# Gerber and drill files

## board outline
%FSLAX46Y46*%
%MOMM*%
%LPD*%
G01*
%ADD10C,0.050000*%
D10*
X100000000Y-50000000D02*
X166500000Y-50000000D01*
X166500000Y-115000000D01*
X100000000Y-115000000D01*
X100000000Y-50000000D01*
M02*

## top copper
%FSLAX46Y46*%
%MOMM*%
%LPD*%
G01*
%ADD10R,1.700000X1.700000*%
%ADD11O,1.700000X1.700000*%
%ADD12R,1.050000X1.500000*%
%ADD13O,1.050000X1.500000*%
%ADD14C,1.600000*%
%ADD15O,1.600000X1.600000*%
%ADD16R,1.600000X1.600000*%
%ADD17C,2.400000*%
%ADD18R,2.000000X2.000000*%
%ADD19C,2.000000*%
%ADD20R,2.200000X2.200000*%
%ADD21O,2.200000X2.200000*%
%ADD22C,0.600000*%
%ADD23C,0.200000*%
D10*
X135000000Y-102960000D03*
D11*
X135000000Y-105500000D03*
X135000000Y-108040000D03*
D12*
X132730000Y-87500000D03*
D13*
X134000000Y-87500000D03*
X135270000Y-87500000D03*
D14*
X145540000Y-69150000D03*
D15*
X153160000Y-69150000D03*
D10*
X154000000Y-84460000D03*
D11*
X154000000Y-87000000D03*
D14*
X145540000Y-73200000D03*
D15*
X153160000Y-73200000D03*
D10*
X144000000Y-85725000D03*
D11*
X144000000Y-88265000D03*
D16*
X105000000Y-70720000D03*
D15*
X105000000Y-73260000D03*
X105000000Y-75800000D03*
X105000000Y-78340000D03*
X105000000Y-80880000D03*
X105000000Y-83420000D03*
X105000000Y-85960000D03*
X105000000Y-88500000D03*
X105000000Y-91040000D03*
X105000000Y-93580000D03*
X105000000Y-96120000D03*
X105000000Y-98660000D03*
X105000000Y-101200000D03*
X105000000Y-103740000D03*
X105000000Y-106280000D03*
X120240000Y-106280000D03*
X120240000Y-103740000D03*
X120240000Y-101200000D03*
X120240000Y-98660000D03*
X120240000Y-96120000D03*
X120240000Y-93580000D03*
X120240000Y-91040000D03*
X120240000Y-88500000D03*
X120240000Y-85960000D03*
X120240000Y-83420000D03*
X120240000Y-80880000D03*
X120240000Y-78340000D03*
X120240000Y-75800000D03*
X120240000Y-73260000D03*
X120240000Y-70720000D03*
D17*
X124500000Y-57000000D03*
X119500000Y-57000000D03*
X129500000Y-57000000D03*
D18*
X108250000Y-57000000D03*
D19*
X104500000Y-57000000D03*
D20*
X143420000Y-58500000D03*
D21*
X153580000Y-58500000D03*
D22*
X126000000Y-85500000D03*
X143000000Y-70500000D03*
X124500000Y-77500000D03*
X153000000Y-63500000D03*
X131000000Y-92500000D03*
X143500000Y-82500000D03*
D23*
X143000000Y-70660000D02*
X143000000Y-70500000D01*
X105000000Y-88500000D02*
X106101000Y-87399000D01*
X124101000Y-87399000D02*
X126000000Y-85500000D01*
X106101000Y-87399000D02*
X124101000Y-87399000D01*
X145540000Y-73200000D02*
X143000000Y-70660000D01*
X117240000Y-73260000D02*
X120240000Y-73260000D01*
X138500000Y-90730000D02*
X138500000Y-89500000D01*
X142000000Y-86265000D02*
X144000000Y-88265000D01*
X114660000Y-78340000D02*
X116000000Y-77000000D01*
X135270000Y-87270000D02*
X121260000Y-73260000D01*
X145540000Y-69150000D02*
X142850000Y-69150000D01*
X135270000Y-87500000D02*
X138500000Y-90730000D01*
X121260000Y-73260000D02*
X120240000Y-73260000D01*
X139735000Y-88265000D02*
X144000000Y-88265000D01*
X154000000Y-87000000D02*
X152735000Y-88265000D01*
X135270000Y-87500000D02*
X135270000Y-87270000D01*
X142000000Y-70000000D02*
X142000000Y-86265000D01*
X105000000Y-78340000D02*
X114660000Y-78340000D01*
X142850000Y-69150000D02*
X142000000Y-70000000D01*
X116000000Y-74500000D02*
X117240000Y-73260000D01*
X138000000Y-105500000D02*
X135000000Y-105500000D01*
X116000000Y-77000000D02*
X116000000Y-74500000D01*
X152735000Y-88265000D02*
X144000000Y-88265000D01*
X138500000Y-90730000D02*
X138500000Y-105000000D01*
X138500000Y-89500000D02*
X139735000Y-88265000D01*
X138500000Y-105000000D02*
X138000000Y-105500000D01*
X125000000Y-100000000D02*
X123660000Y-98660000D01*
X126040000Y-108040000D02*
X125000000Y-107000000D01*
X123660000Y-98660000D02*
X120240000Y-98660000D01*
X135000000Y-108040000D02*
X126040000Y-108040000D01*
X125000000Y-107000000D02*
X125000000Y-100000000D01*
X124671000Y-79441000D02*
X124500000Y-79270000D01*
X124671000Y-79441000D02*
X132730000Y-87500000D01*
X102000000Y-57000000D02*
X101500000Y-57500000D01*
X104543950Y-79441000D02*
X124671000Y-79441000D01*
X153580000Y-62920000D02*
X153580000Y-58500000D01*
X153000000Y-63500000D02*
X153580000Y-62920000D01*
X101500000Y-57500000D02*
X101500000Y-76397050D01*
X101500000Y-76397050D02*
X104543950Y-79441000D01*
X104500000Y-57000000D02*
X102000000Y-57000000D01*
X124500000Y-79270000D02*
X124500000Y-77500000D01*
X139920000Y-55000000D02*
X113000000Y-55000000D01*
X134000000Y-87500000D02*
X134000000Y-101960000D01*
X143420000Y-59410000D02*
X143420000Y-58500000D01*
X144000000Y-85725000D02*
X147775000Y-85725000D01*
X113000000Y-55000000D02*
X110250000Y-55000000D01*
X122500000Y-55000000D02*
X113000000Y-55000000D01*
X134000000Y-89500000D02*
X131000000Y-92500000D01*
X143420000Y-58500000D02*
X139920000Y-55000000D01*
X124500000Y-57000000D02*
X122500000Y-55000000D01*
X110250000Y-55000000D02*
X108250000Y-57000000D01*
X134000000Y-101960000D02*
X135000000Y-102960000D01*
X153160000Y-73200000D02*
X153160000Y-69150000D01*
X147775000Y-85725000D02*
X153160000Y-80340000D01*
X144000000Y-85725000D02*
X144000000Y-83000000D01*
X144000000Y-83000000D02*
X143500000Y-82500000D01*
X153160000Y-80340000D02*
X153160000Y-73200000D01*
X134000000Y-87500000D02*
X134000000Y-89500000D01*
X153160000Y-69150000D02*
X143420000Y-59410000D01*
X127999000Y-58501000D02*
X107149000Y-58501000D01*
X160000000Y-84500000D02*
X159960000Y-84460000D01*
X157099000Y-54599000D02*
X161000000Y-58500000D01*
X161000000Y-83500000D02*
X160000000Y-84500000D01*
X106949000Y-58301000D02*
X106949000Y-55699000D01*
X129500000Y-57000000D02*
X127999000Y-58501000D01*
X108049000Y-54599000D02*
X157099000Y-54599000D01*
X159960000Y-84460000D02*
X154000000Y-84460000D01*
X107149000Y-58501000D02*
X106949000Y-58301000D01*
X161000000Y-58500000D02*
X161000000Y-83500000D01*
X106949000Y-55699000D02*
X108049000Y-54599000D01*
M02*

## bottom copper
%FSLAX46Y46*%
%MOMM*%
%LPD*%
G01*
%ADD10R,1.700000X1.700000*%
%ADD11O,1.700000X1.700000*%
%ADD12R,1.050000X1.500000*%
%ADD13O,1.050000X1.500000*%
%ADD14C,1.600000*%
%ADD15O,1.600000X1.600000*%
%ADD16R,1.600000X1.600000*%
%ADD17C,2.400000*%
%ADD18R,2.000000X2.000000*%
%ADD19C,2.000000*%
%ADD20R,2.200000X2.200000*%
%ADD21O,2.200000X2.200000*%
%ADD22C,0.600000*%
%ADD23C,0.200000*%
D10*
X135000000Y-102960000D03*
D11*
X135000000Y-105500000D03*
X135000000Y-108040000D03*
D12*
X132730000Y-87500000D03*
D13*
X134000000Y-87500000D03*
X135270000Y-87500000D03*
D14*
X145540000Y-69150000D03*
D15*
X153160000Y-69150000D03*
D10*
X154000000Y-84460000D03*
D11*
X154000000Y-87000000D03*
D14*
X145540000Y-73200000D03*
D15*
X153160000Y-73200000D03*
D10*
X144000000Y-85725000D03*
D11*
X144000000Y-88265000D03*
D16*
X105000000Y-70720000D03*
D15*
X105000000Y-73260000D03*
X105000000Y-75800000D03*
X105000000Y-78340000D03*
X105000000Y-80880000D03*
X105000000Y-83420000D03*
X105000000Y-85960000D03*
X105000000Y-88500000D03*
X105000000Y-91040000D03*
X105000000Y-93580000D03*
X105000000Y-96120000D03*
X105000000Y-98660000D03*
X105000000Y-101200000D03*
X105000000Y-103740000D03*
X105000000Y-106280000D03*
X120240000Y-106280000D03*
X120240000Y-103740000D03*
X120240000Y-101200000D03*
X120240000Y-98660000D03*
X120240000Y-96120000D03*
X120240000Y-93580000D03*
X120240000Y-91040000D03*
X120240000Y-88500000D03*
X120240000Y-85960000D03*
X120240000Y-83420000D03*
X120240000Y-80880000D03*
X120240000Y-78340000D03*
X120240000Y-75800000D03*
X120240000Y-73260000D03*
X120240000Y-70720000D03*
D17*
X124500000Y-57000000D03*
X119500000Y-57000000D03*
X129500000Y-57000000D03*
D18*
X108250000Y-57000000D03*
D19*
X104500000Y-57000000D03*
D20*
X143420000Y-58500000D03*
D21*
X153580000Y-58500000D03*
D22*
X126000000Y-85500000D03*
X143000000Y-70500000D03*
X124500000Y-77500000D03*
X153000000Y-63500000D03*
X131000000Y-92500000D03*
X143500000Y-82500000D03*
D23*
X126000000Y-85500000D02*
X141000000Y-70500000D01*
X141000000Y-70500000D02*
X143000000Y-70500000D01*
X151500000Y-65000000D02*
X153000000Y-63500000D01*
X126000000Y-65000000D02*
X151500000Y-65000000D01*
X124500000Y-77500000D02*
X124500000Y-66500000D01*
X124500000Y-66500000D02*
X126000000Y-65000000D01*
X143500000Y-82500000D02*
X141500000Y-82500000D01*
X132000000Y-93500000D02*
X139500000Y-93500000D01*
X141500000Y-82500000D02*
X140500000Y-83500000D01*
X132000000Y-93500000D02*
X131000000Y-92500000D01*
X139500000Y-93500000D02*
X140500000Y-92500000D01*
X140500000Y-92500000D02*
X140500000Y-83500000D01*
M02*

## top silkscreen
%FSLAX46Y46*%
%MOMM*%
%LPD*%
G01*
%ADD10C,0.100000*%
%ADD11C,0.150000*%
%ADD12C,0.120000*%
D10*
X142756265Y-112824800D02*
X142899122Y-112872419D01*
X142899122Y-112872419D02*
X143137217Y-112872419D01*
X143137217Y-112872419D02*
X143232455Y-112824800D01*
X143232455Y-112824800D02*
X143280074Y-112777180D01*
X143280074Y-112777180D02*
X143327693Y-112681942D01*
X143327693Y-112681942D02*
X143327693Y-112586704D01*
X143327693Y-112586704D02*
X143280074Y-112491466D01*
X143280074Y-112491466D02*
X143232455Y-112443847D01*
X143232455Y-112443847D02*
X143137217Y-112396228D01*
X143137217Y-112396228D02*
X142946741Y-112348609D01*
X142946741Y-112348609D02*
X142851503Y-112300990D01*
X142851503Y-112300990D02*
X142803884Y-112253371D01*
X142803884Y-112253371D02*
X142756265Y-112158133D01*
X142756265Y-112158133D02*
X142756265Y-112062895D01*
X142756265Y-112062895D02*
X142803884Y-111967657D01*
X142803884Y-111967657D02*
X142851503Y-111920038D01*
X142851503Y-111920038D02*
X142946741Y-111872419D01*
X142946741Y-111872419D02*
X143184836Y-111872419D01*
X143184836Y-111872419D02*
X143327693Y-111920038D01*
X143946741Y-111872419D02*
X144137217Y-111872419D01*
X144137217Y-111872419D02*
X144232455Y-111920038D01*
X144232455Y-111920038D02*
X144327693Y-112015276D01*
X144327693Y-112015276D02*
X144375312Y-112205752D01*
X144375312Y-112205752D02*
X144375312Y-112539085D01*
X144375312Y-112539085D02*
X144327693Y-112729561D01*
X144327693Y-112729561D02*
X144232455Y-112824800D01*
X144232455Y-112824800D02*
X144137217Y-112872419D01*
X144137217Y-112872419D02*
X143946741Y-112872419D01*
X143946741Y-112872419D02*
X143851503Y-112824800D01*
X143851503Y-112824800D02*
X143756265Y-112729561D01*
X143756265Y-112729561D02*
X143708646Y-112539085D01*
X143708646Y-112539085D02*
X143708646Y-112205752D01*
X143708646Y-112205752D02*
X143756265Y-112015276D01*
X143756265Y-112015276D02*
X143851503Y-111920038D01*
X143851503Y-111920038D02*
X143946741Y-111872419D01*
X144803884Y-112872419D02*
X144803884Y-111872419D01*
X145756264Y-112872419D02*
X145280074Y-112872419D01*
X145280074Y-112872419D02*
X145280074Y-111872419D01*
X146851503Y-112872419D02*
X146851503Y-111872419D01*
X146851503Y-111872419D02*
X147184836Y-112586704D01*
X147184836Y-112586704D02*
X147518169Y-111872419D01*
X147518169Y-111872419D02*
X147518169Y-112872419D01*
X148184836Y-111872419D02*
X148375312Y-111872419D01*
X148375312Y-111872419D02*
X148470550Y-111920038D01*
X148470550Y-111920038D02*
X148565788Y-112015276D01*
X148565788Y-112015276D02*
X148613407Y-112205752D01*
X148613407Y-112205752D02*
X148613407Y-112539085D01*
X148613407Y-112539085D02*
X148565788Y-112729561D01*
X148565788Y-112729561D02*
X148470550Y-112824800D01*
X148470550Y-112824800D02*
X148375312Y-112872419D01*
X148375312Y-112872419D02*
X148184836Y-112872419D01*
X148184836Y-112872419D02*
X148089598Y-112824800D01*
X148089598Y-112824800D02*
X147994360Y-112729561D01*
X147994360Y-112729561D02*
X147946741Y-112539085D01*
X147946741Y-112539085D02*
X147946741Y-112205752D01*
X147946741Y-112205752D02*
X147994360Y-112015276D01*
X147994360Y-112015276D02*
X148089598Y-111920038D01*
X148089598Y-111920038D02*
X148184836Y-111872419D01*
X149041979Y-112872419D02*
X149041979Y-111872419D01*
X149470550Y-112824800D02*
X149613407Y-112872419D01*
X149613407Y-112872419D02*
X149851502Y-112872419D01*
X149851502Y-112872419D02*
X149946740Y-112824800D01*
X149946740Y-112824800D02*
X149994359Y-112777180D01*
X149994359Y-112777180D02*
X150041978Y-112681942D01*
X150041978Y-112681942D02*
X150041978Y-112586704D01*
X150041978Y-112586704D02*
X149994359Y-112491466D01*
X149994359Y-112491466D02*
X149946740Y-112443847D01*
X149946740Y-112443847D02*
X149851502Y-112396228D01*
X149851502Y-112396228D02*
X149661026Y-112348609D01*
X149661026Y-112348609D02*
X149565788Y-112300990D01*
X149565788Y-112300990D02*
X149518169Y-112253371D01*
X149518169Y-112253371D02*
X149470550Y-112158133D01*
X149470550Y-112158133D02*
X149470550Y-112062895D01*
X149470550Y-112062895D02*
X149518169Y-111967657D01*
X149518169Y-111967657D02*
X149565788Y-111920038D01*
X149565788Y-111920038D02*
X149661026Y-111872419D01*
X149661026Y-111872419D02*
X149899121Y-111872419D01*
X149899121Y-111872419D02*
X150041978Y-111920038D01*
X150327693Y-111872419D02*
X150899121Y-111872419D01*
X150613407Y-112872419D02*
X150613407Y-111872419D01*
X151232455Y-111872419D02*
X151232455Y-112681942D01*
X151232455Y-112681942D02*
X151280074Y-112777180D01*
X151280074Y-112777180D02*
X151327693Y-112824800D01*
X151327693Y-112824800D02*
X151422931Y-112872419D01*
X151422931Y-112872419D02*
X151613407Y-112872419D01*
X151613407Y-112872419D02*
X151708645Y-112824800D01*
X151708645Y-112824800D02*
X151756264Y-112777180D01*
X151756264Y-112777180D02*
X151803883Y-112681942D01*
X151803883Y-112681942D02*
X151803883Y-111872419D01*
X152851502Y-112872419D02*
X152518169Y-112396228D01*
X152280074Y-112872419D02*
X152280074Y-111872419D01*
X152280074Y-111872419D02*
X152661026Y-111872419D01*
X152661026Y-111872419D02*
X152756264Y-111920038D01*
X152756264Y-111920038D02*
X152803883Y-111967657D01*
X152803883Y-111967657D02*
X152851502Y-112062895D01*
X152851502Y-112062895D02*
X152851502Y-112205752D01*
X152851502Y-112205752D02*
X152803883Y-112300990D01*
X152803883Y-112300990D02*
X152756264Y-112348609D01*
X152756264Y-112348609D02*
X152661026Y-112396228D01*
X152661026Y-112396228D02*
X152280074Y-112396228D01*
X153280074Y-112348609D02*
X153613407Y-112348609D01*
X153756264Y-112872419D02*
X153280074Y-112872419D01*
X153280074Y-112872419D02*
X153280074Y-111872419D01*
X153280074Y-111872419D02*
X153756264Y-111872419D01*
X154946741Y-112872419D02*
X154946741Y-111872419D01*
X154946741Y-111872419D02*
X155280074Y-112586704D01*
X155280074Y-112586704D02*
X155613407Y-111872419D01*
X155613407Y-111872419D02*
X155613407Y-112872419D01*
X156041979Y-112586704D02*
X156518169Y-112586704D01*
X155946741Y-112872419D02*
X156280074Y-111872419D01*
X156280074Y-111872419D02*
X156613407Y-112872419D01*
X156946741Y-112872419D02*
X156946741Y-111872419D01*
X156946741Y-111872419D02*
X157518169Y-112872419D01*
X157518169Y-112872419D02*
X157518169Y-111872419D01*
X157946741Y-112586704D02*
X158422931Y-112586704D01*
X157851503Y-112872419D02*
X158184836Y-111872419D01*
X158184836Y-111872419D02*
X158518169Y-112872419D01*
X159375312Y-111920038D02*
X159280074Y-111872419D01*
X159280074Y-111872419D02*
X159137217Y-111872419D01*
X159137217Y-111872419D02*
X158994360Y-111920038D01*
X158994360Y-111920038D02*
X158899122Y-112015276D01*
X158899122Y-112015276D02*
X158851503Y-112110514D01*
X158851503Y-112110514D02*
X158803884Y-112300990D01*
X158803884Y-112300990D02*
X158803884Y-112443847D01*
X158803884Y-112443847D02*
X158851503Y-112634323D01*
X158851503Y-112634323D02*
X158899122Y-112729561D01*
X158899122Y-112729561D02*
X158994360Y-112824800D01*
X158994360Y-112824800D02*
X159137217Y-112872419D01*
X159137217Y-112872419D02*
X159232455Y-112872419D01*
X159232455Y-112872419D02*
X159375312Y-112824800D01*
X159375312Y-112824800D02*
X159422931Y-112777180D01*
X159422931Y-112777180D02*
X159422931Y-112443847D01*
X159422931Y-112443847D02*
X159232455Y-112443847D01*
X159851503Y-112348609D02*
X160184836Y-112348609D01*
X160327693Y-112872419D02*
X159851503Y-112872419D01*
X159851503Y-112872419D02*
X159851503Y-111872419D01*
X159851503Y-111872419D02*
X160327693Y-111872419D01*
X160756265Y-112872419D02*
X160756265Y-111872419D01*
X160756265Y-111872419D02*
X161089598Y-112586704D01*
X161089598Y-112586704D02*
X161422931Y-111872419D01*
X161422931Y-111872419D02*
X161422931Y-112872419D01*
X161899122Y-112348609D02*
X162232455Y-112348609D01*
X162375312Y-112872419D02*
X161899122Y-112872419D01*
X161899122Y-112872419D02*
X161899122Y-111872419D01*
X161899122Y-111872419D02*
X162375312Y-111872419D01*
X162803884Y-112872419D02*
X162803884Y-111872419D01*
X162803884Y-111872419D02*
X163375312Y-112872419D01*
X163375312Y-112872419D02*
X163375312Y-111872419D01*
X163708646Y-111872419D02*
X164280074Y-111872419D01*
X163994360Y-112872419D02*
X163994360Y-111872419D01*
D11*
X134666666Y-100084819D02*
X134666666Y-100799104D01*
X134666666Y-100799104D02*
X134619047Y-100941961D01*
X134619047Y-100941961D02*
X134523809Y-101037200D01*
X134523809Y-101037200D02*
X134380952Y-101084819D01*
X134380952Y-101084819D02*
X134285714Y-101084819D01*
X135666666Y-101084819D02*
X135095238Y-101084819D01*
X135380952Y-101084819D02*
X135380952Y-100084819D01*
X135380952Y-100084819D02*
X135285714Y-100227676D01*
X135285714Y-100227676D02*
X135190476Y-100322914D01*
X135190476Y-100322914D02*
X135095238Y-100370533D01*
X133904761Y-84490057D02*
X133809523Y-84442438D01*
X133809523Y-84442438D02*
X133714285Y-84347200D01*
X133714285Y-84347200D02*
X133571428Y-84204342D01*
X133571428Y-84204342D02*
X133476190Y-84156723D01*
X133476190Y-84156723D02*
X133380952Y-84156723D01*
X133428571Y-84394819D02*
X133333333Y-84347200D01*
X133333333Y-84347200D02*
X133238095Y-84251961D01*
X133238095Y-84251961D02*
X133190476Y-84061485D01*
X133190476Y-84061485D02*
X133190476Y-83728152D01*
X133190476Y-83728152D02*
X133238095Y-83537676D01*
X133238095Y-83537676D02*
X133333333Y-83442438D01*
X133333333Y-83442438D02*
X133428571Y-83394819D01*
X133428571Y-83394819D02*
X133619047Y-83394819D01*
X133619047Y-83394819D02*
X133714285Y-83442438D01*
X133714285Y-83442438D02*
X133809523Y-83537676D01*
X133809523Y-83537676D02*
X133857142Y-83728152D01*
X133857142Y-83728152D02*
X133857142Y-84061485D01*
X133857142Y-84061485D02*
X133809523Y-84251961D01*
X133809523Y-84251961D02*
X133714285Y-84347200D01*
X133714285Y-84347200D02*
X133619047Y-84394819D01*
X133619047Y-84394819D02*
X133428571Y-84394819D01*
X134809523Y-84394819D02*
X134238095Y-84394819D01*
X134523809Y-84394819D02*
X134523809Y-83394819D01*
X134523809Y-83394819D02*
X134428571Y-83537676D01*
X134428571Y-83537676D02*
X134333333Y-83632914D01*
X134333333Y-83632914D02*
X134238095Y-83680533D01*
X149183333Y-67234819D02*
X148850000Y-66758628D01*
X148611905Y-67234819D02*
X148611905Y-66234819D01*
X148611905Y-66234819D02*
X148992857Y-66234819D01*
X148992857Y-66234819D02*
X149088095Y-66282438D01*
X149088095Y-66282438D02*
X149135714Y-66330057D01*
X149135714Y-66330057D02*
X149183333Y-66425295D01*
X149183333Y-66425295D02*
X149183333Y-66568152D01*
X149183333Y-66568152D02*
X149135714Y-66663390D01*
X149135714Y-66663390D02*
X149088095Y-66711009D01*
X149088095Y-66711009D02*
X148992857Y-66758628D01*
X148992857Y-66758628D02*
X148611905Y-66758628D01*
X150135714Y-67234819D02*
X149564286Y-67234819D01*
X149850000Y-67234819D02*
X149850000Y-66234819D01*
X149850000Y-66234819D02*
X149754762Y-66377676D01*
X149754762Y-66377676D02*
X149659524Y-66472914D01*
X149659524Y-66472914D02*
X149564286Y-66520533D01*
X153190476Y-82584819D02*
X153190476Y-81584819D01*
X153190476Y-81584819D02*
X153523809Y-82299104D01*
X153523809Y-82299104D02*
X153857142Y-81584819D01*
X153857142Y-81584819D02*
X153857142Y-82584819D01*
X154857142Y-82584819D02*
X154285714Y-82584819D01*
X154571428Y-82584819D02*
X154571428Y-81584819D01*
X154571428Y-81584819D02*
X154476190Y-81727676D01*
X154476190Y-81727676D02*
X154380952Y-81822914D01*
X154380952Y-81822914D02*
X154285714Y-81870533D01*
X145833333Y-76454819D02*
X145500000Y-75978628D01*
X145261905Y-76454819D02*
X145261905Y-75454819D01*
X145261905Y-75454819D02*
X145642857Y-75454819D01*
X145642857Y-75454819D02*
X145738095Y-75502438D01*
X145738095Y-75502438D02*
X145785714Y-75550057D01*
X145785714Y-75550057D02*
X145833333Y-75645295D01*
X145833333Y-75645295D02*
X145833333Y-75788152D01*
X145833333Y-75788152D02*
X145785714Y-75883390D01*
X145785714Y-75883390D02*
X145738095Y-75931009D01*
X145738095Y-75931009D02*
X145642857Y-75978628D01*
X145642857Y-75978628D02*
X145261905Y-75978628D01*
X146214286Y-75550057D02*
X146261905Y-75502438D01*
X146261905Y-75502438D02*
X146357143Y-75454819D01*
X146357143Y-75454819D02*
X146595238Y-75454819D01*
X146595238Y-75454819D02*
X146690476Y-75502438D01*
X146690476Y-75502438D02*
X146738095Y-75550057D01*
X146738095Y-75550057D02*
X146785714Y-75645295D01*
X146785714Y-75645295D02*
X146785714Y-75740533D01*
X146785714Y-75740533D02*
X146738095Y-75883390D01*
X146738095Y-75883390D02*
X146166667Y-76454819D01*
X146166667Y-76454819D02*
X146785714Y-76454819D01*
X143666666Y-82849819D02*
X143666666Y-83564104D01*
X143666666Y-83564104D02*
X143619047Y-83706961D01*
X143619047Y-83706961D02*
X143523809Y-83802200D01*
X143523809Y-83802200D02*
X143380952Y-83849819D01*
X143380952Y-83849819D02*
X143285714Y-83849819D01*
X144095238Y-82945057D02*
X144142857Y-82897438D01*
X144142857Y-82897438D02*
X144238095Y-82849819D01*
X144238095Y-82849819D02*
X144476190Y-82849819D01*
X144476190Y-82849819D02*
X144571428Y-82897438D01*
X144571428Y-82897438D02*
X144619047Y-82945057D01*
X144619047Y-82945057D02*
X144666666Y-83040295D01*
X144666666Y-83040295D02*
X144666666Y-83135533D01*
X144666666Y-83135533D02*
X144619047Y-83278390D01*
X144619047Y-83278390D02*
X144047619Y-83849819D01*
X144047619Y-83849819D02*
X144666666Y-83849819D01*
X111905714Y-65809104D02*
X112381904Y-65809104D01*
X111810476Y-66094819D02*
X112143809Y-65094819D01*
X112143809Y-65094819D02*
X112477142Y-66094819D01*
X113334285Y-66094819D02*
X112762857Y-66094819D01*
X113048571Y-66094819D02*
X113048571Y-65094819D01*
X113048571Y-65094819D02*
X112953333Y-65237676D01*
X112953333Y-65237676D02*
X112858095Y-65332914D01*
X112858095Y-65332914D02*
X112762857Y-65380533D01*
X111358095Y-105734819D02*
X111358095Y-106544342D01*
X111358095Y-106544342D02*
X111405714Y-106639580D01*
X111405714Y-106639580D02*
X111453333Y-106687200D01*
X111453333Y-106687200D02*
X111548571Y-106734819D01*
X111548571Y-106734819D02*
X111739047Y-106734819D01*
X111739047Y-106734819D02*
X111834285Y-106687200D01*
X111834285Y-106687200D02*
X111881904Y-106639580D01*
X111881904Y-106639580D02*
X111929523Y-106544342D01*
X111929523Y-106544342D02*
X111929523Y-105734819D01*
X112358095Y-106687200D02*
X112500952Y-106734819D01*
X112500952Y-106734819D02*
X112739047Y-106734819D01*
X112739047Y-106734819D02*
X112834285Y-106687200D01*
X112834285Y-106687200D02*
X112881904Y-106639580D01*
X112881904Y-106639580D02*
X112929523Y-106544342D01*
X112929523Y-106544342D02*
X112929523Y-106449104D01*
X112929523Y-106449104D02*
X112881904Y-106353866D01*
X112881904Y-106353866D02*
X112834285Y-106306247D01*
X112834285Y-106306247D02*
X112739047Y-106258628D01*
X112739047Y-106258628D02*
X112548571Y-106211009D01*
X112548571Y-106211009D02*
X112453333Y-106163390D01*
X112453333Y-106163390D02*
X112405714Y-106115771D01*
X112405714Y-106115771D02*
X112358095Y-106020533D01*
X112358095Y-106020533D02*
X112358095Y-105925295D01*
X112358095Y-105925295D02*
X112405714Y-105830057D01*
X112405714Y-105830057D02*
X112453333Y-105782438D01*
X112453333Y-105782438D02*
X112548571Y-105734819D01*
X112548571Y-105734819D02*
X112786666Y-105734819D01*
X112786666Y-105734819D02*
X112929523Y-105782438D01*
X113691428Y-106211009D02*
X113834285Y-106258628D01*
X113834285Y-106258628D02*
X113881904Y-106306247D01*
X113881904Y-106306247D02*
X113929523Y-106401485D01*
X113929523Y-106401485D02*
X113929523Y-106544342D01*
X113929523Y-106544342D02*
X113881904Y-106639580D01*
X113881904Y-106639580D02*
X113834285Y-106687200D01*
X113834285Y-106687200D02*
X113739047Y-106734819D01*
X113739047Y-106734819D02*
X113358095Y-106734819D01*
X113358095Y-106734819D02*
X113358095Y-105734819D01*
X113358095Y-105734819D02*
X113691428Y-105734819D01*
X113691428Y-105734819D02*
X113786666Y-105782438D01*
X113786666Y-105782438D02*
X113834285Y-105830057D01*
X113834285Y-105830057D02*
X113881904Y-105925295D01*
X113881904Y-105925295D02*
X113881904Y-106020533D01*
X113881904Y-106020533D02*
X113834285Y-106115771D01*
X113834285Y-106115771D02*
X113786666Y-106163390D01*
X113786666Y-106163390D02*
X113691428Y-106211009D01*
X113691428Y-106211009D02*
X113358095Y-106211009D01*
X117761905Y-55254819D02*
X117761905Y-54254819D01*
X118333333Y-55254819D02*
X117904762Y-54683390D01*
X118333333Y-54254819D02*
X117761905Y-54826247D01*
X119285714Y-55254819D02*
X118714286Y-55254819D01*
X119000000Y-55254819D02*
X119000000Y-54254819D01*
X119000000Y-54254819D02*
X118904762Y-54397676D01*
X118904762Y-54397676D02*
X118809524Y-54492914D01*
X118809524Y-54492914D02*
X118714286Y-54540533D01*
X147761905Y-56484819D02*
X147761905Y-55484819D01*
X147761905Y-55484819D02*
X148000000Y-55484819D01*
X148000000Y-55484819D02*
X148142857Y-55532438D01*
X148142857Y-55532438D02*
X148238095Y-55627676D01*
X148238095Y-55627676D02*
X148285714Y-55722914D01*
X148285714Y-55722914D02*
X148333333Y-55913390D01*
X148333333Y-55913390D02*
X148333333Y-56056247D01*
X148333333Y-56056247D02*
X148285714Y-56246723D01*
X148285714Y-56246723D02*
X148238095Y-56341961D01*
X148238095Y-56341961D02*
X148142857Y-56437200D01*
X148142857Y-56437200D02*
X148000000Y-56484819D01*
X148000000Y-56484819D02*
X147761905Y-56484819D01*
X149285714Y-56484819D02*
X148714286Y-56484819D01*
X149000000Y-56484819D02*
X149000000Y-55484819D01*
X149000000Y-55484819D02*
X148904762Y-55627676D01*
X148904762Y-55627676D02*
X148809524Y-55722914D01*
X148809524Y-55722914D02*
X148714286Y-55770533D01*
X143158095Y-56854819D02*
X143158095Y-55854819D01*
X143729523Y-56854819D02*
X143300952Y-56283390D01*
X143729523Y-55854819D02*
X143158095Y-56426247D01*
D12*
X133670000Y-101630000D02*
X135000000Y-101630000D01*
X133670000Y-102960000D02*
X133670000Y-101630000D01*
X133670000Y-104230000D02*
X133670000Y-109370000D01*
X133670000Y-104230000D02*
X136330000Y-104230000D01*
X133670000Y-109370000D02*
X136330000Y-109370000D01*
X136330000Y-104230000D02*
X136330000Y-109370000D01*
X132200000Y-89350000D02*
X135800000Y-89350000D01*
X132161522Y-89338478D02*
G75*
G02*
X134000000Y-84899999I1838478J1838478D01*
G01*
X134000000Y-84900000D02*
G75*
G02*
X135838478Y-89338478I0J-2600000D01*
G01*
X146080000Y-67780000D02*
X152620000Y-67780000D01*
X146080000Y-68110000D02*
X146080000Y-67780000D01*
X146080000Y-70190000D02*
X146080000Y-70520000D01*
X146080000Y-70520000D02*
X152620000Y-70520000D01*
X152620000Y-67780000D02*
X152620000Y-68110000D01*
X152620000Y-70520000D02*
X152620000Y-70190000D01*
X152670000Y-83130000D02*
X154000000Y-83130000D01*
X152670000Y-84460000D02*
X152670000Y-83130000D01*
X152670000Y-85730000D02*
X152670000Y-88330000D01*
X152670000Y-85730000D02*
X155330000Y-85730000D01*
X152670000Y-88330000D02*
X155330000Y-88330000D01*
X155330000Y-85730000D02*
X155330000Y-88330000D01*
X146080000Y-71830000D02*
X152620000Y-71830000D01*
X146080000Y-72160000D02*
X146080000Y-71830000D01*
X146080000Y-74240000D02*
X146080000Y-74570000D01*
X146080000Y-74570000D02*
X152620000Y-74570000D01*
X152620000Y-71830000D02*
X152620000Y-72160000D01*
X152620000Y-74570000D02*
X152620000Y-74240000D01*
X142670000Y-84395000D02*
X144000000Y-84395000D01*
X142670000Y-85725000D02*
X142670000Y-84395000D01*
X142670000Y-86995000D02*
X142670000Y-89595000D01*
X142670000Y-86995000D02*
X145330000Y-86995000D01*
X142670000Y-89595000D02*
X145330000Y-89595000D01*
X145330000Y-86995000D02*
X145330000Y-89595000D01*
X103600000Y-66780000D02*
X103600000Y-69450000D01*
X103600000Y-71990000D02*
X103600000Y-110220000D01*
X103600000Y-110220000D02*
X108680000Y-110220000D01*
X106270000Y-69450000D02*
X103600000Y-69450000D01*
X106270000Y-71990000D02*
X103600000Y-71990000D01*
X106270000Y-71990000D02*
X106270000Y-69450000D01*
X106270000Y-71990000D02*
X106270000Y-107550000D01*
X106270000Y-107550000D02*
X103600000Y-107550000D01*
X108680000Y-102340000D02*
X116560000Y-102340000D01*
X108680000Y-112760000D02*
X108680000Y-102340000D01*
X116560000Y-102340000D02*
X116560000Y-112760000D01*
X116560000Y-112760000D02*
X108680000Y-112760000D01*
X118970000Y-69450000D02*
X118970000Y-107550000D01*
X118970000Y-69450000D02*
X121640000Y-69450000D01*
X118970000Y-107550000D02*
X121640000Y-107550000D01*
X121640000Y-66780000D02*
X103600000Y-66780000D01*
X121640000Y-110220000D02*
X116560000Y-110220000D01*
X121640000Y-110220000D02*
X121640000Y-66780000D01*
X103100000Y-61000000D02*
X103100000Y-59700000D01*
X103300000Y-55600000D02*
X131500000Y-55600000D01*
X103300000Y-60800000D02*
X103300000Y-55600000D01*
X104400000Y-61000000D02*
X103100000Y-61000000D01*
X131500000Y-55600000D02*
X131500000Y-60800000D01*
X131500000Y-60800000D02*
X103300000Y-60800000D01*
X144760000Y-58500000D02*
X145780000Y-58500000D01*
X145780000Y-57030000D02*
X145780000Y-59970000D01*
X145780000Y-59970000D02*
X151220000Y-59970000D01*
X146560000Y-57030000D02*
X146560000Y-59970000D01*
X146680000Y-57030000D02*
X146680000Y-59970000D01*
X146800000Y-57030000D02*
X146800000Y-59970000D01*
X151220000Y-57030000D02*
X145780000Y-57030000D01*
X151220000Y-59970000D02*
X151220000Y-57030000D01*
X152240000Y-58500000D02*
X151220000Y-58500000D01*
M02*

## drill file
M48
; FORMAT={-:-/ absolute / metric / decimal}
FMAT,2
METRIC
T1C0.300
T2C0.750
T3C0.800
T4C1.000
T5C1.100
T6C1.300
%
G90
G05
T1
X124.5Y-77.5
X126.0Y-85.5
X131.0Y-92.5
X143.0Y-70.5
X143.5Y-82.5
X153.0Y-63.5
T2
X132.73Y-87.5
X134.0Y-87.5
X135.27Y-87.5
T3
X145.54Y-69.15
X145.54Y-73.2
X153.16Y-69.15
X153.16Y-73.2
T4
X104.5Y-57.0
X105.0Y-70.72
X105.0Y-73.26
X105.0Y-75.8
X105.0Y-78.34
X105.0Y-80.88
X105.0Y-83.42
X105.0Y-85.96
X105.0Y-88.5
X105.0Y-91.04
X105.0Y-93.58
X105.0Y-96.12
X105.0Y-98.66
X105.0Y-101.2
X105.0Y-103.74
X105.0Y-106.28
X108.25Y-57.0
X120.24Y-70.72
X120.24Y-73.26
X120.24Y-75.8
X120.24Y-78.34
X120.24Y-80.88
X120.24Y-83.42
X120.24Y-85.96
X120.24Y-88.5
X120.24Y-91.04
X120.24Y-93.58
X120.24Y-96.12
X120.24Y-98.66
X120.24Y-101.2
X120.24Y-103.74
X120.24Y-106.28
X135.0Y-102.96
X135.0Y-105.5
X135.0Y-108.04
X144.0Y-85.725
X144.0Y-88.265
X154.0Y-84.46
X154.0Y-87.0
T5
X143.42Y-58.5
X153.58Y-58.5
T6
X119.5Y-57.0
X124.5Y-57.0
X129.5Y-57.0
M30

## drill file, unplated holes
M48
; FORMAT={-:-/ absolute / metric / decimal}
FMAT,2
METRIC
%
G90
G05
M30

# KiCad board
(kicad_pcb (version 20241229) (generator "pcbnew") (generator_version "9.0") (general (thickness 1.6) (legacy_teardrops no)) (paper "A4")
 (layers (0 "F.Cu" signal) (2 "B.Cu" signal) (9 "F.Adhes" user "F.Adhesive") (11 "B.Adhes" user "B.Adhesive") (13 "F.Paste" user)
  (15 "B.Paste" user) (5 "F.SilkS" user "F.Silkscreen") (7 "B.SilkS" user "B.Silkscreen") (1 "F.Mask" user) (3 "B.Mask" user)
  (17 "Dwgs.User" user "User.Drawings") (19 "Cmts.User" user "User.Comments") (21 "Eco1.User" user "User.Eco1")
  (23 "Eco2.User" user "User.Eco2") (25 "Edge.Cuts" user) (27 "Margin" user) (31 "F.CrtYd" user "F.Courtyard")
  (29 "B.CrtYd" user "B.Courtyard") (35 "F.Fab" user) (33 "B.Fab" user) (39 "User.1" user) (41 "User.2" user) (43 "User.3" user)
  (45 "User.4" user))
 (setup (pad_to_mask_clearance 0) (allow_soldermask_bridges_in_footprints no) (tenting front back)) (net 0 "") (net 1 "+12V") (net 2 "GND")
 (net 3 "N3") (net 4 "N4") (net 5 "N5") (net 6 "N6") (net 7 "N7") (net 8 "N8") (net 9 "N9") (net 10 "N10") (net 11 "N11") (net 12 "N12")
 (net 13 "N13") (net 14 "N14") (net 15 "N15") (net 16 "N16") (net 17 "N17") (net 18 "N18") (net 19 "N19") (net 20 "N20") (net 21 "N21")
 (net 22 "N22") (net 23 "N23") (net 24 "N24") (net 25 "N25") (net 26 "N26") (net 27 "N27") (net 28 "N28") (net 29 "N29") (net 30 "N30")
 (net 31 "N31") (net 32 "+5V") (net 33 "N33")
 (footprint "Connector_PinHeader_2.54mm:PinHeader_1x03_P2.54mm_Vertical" (layer "F.Cu") (at 135 102.96)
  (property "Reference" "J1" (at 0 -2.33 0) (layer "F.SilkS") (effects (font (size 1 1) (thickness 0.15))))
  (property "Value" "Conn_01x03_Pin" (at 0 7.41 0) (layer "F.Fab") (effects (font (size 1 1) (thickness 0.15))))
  (fp_line (start -1.33 -1.33) (end 0 -1.33) (stroke (width 0.12) (type solid)) (layer "F.SilkS"))
  (fp_line (start -1.33 0) (end -1.33 -1.33) (stroke (width 0.12) (type solid)) (layer "F.SilkS"))
  (fp_line (start -1.33 1.27) (end -1.33 6.41) (stroke (width 0.12) (type solid)) (layer "F.SilkS"))
  (fp_line (start -1.33 1.27) (end 1.33 1.27) (stroke (width 0.12) (type solid)) (layer "F.SilkS"))
  (fp_line (start -1.33 6.41) (end 1.33 6.41) (stroke (width 0.12) (type solid)) (layer "F.SilkS"))
  (fp_line (start 1.33 1.27) (end 1.33 6.41) (stroke (width 0.12) (type solid)) (layer "F.SilkS"))
  (pad "1" thru_hole rect (at 0 0) (size 1.7 1.7) (drill 1) (layers "*.Cu" "*.Mask") (remove_unused_layers no) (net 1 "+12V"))
  (pad "2" thru_hole oval (at 0 2.54) (size 1.7 1.7) (drill 1) (layers "*.Cu" "*.Mask") (remove_unused_layers no) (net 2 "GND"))
  (pad "3" thru_hole oval (at 0 5.08) (size 1.7 1.7) (drill 1) (layers "*.Cu" "*.Mask") (remove_unused_layers no) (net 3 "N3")))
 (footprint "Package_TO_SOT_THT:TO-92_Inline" (layer "F.Cu") (at 132.73 87.5)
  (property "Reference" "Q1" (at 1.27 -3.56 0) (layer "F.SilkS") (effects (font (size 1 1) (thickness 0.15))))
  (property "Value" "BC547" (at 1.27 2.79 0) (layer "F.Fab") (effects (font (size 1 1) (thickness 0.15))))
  (fp_line (start -0.53 1.85) (end 3.07 1.85) (stroke (width 0.12) (type solid)) (layer "F.SilkS"))
  (fp_arc (start -0.568478 1.838478) (mid -1.132087 -0.994977) (end 1.27 -2.6) (stroke (width 0.12) (type solid)) (layer "F.SilkS"))
  (fp_arc (start 1.27 -2.6) (mid 3.672087 -0.994977) (end 3.108478 1.838478) (stroke (width 0.12) (type solid)) (layer "F.SilkS"))
  (pad "1" thru_hole rect (at 0 0) (size 1.05 1.5) (drill 0.75) (layers "*.Cu" "*.Mask") (remove_unused_layers no) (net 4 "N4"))
  (pad "2" thru_hole oval (at 1.27 0) (size 1.05 1.5) (drill 0.75) (layers "*.Cu" "*.Mask") (remove_unused_layers no) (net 1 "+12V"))
  (pad "3" thru_hole oval (at 2.54 0) (size 1.05 1.5) (drill 0.75) (layers "*.Cu" "*.Mask") (remove_unused_layers no) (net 2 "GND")))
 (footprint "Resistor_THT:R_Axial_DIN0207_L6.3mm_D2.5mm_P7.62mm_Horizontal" (layer "F.Cu") (at 145.54 69.15)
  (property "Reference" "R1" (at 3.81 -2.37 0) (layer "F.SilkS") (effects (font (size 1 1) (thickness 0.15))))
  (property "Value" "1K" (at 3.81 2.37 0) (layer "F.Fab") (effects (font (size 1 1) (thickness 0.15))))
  (fp_line (start 0.54 -1.37) (end 7.08 -1.37) (stroke (width 0.12) (type solid)) (layer "F.SilkS"))
  (fp_line (start 0.54 -1.04) (end 0.54 -1.37) (stroke (width 0.12) (type solid)) (layer "F.SilkS"))
  (fp_line (start 0.54 1.04) (end 0.54 1.37) (stroke (width 0.12) (type solid)) (layer "F.SilkS"))
  (fp_line (start 0.54 1.37) (end 7.08 1.37) (stroke (width 0.12) (type solid)) (layer "F.SilkS"))
  (fp_line (start 7.08 -1.37) (end 7.08 -1.04) (stroke (width 0.12) (type solid)) (layer "F.SilkS"))
  (fp_line (start 7.08 1.37) (end 7.08 1.04) (stroke (width 0.12) (type solid)) (layer "F.SilkS"))
  (pad "1" thru_hole circle (at 0 0) (size 1.6 1.6) (drill 0.8) (layers "*.Cu" "*.Mask") (remove_unused_layers no) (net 2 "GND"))
  (pad "2" thru_hole oval (at 7.62 0) (size 1.6 1.6) (drill 0.8) (layers "*.Cu" "*.Mask") (remove_unused_layers no) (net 1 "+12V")))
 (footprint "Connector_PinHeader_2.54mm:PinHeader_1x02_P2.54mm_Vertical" (layer "F.Cu") (at 154 84.46)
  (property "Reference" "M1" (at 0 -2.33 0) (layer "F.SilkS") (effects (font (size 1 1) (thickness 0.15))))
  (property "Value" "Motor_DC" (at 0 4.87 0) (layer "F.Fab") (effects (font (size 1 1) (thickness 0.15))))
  (fp_line (start -1.33 -1.33) (end 0 -1.33) (stroke (width 0.12) (type solid)) (layer "F.SilkS"))
  (fp_line (start -1.33 0) (end -1.33 -1.33) (stroke (width 0.12) (type solid)) (layer "F.SilkS"))
  (fp_line (start -1.33 1.27) (end -1.33 3.87) (stroke (width 0.12) (type solid)) (layer "F.SilkS"))
  (fp_line (start -1.33 1.27) (end 1.33 1.27) (stroke (width 0.12) (type solid)) (layer "F.SilkS"))
  (fp_line (start -1.33 3.87) (end 1.33 3.87) (stroke (width 0.12) (type solid)) (layer "F.SilkS"))
  (fp_line (start 1.33 1.27) (end 1.33 3.87) (stroke (width 0.12) (type solid)) (layer "F.SilkS"))
  (pad "1" thru_hole rect (at 0 0) (size 1.7 1.7) (drill 1) (layers "*.Cu" "*.Mask") (remove_unused_layers no) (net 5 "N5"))
  (pad "2" thru_hole oval (at 0 2.54) (size 1.7 1.7) (drill 1) (layers "*.Cu" "*.Mask") (remove_unused_layers no) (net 2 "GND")))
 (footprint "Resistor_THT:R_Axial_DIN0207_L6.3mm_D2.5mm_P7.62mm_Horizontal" (layer "F.Cu") (at 145.54 73.2)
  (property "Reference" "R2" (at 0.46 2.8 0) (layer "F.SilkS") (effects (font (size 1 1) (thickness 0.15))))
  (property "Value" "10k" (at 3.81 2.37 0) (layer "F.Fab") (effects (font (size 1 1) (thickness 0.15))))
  (fp_line (start 0.54 -1.37) (end 7.08 -1.37) (stroke (width 0.12) (type solid)) (layer "F.SilkS"))
  (fp_line (start 0.54 -1.04) (end 0.54 -1.37) (stroke (width 0.12) (type solid)) (layer "F.SilkS"))
  (fp_line (start 0.54 1.04) (end 0.54 1.37) (stroke (width 0.12) (type solid)) (layer "F.SilkS"))
  (fp_line (start 0.54 1.37) (end 7.08 1.37) (stroke (width 0.12) (type solid)) (layer "F.SilkS"))
  (fp_line (start 7.08 -1.37) (end 7.08 -1.04) (stroke (width 0.12) (type solid)) (layer "F.SilkS"))
  (fp_line (start 7.08 1.37) (end 7.08 1.04) (stroke (width 0.12) (type solid)) (layer "F.SilkS"))
  (pad "1" thru_hole circle (at 0 0) (size 1.6 1.6) (drill 0.8) (layers "*.Cu" "*.Mask") (remove_unused_layers no) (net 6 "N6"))
  (pad "2" thru_hole oval (at 7.62 0) (size 1.6 1.6) (drill 0.8) (layers "*.Cu" "*.Mask") (remove_unused_layers no) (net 1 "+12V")))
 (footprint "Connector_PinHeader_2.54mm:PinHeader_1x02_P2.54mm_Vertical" (layer "F.Cu") (at 144 85.725)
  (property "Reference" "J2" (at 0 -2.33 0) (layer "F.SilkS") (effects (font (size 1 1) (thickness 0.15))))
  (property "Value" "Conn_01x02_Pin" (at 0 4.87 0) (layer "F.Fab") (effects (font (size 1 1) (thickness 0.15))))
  (fp_line (start -1.33 -1.33) (end 0 -1.33) (stroke (width 0.12) (type solid)) (layer "F.SilkS"))
  (fp_line (start -1.33 0) (end -1.33 -1.33) (stroke (width 0.12) (type solid)) (layer "F.SilkS"))
  (fp_line (start -1.33 1.27) (end -1.33 3.87) (stroke (width 0.12) (type solid)) (layer "F.SilkS"))
  (fp_line (start -1.33 1.27) (end 1.33 1.27) (stroke (width 0.12) (type solid)) (layer "F.SilkS"))
  (fp_line (start -1.33 3.87) (end 1.33 3.87) (stroke (width 0.12) (type solid)) (layer "F.SilkS"))
  (fp_line (start 1.33 1.27) (end 1.33 3.87) (stroke (width 0.12) (type solid)) (layer "F.SilkS"))
  (pad "1" thru_hole rect (at 0 0) (size 1.7 1.7) (drill 1) (layers "*.Cu" "*.Mask") (remove_unused_layers no) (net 1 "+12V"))
  (pad "2" thru_hole oval (at 0 2.54) (size 1.7 1.7) (drill 1) (layers "*.Cu" "*.Mask") (remove_unused_layers no) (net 2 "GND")))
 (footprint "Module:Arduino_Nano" (layer "F.Cu") (at 105 70.72)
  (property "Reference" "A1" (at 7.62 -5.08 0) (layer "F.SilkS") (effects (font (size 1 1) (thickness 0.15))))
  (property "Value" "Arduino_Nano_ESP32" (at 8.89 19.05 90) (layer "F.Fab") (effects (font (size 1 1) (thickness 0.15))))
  (fp_line (start -1.4 -3.94) (end -1.4 -1.27) (stroke (width 0.12) (type solid)) (layer "F.SilkS"))
  (fp_line (start -1.4 1.27) (end -1.4 39.5) (stroke (width 0.12) (type solid)) (layer "F.SilkS"))
  (fp_line (start -1.4 39.5) (end 3.68 39.5) (stroke (width 0.12) (type solid)) (layer "F.SilkS"))
  (fp_line (start 1.27 -1.27) (end -1.4 -1.27) (stroke (width 0.12) (type solid)) (layer "F.SilkS"))
  (fp_line (start 1.27 1.27) (end -1.4 1.27) (stroke (width 0.12) (type solid)) (layer "F.SilkS"))
  (fp_line (start 1.27 1.27) (end 1.27 -1.27) (stroke (width 0.12) (type solid)) (layer "F.SilkS"))
  (fp_line (start 1.27 1.27) (end 1.27 36.83) (stroke (width 0.12) (type solid)) (layer "F.SilkS"))
  (fp_line (start 1.27 36.83) (end -1.4 36.83) (stroke (width 0.12) (type solid)) (layer "F.SilkS"))
  (fp_line (start 3.68 31.62) (end 11.56 31.62) (stroke (width 0.12) (type solid)) (layer "F.SilkS"))
  (fp_line (start 3.68 42.04) (end 3.68 31.62) (stroke (width 0.12) (type solid)) (layer "F.SilkS"))
  (fp_line (start 11.56 31.62) (end 11.56 42.04) (stroke (width 0.12) (type solid)) (layer "F.SilkS"))
  (fp_line (start 11.56 42.04) (end 3.68 42.04) (stroke (width 0.12) (type solid)) (layer "F.SilkS"))
  (fp_line (start 13.97 -1.27) (end 13.97 36.83) (stroke (width 0.12) (type solid)) (layer "F.SilkS"))
  (fp_line (start 13.97 -1.27) (end 16.64 -1.27) (stroke (width 0.12) (type solid)) (layer "F.SilkS"))
  (fp_line (start 13.97 36.83) (end 16.64 36.83) (stroke (width 0.12) (type solid)) (layer "F.SilkS"))
  (fp_line (start 16.64 -3.94) (end -1.4 -3.94) (stroke (width 0.12) (type solid)) (layer "F.SilkS"))
  (fp_line (start 16.64 39.5) (end 11.56 39.5) (stroke (width 0.12) (type solid)) (layer "F.SilkS"))
  (fp_line (start 16.64 39.5) (end 16.64 -3.94) (stroke (width 0.12) (type solid)) (layer "F.SilkS"))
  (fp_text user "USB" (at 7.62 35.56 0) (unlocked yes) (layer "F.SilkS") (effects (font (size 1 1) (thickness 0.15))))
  (pad "1" thru_hole rect (at 0 0) (size 1.6 1.6) (drill 1) (layers "*.Cu" "*.Mask") (remove_unused_layers no) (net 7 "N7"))
  (pad "2" thru_hole oval (at 0 2.54) (size 1.6 1.6) (drill 1) (layers "*.Cu" "*.Mask") (remove_unused_layers no) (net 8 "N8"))
  (pad "3" thru_hole oval (at 0 5.08) (size 1.6 1.6) (drill 1) (layers "*.Cu" "*.Mask") (remove_unused_layers no) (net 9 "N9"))
  (pad "4" thru_hole oval (at 0 7.62) (size 1.6 1.6) (drill 1) (layers "*.Cu" "*.Mask") (remove_unused_layers no) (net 2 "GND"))
  (pad "5" thru_hole oval (at 0 10.16) (size 1.6 1.6) (drill 1) (layers "*.Cu" "*.Mask") (remove_unused_layers no) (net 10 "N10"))
  (pad "6" thru_hole oval (at 0 12.7) (size 1.6 1.6) (drill 1) (layers "*.Cu" "*.Mask") (remove_unused_layers no) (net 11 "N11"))
  (pad "7" thru_hole oval (at 0 15.24) (size 1.6 1.6) (drill 1) (layers "*.Cu" "*.Mask") (remove_unused_layers no) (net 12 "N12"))
  (pad "8" thru_hole oval (at 0 17.78) (size 1.6 1.6) (drill 1) (layers "*.Cu" "*.Mask") (remove_unused_layers no) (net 6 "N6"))
  (pad "9" thru_hole oval (at 0 20.32) (size 1.6 1.6) (drill 1) (layers "*.Cu" "*.Mask") (remove_unused_layers no) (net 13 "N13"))
  (pad "10" thru_hole oval (at 0 22.86) (size 1.6 1.6) (drill 1) (layers "*.Cu" "*.Mask") (remove_unused_layers no) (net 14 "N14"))
  (pad "11" thru_hole oval (at 0 25.4) (size 1.6 1.6) (drill 1) (layers "*.Cu" "*.Mask") (remove_unused_layers no) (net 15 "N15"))
  (pad "12" thru_hole oval (at 0 27.94) (size 1.6 1.6) (drill 1) (layers "*.Cu" "*.Mask") (remove_unused_layers no) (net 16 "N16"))
  (pad "13" thru_hole oval (at 0 30.48) (size 1.6 1.6) (drill 1) (layers "*.Cu" "*.Mask") (remove_unused_layers no) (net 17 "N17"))
  (pad "14" thru_hole oval (at 0 33.02) (size 1.6 1.6) (drill 1) (layers "*.Cu" "*.Mask") (remove_unused_layers no) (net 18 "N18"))
  (pad "15" thru_hole oval (at 0 35.56) (size 1.6 1.6) (drill 1) (layers "*.Cu" "*.Mask") (remove_unused_layers no) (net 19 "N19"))
  (pad "16" thru_hole oval (at 15.24 35.56) (size 1.6 1.6) (drill 1) (layers "*.Cu" "*.Mask") (remove_unused_layers no) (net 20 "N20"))
  (pad "17" thru_hole oval (at 15.24 33.02) (size 1.6 1.6) (drill 1) (layers "*.Cu" "*.Mask") (remove_unused_layers no) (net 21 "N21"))
  (pad "18" thru_hole oval (at 15.24 30.48) (size 1.6 1.6) (drill 1) (layers "*.Cu" "*.Mask") (remove_unused_layers no) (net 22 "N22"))
  (pad "19" thru_hole oval (at 15.24 27.94) (size 1.6 1.6) (drill 1) (layers "*.Cu" "*.Mask") (remove_unused_layers no) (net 3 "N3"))
  (pad "20" thru_hole oval (at 15.24 25.4) (size 1.6 1.6) (drill 1) (layers "*.Cu" "*.Mask") (remove_unused_layers no) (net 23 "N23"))
  (pad "21" thru_hole oval (at 15.24 22.86) (size 1.6 1.6) (drill 1) (layers "*.Cu" "*.Mask") (remove_unused_layers no) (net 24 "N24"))
  (pad "22" thru_hole oval (at 15.24 20.32) (size 1.6 1.6) (drill 1) (layers "*.Cu" "*.Mask") (remove_unused_layers no) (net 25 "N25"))
  (pad "23" thru_hole oval (at 15.24 17.78) (size 1.6 1.6) (drill 1) (layers "*.Cu" "*.Mask") (remove_unused_layers no) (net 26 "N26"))
  (pad "24" thru_hole oval (at 15.24 15.24) (size 1.6 1.6) (drill 1) (layers "*.Cu" "*.Mask") (remove_unused_layers no) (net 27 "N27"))
  (pad "25" thru_hole oval (at 15.24 12.7) (size 1.6 1.6) (drill 1) (layers "*.Cu" "*.Mask") (remove_unused_layers no) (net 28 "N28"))
  (pad "26" thru_hole oval (at 15.24 10.16) (size 1.6 1.6) (drill 1) (layers "*.Cu" "*.Mask") (remove_unused_layers no) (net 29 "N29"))
  (pad "27" thru_hole oval (at 15.24 7.62) (size 1.6 1.6) (drill 1) (layers "*.Cu" "*.Mask") (remove_unused_layers no) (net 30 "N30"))
  (pad "28" thru_hole oval (at 15.24 5.08) (size 1.6 1.6) (drill 1) (layers "*.Cu" "*.Mask") (remove_unused_layers no) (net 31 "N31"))
  (pad "29" thru_hole oval (at 15.24 2.54) (size 1.6 1.6) (drill 1) (layers "*.Cu" "*.Mask") (remove_unused_layers no) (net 2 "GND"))
  (pad "30" thru_hole oval (at 15.24 0) (size 1.6 1.6) (drill 1) (layers "*.Cu" "*.Mask") (remove_unused_layers no) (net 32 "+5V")))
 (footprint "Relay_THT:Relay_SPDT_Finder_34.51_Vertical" (layer "F.Cu") (at 108.25 57)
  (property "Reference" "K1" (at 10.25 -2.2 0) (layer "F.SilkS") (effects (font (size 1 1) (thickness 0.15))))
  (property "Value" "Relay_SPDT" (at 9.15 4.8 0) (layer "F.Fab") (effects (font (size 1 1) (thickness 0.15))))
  (fp_line (start -5.15 4) (end -5.15 2.7) (stroke (width 0.12) (type solid)) (layer "F.SilkS"))
  (fp_line (start -4.95 -1.4) (end 23.25 -1.4) (stroke (width 0.12) (type solid)) (layer "F.SilkS"))
  (fp_line (start -4.95 3.8) (end -4.95 -1.4) (stroke (width 0.12) (type solid)) (layer "F.SilkS"))
  (fp_line (start -3.85 4) (end -5.15 4) (stroke (width 0.12) (type solid)) (layer "F.SilkS"))
  (fp_line (start 23.25 -1.4) (end 23.25 3.8) (stroke (width 0.12) (type solid)) (layer "F.SilkS"))
  (fp_line (start 23.25 3.8) (end -4.95 3.8) (stroke (width 0.12) (type solid)) (layer "F.SilkS"))
  (pad "11" thru_hole circle (at 16.25 0) (size 2.4 2.4) (drill 1.3) (layers "*.Cu" "*.Mask") (remove_unused_layers no) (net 1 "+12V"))
  (pad "12" thru_hole circle (at 11.25 0) (size 2.4 2.4) (drill 1.3) (layers "*.Cu" "*.Mask") (remove_unused_layers no) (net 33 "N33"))
  (pad "14" thru_hole circle (at 21.25 0) (size 2.4 2.4) (drill 1.3) (layers "*.Cu" "*.Mask") (remove_unused_layers no) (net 5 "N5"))
  (pad "A1" thru_hole rect (at 0 0) (size 2 2) (drill 1) (layers "*.Cu" "*.Mask") (remove_unused_layers no) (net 1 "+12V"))
  (pad "A2" thru_hole circle (at -3.75 0) (size 2 2) (drill 1) (layers "*.Cu" "*.Mask") (remove_unused_layers no) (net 4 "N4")))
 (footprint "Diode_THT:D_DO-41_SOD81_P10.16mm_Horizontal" (layer "F.Cu") (at 143.42 58.5)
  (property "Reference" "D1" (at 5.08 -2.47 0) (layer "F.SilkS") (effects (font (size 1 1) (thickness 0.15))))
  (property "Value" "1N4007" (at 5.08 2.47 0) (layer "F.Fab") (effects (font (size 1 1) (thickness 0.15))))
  (fp_line (start 1.34 0) (end 2.36 0) (stroke (width 0.12) (type solid)) (layer "F.SilkS"))
  (fp_line (start 2.36 -1.47) (end 2.36 1.47) (stroke (width 0.12) (type solid)) (layer "F.SilkS"))
  (fp_line (start 2.36 1.47) (end 7.8 1.47) (stroke (width 0.12) (type solid)) (layer "F.SilkS"))
  (fp_line (start 3.14 -1.47) (end 3.14 1.47) (stroke (width 0.12) (type solid)) (layer "F.SilkS"))
  (fp_line (start 3.26 -1.47) (end 3.26 1.47) (stroke (width 0.12) (type solid)) (layer "F.SilkS"))
  (fp_line (start 3.38 -1.47) (end 3.38 1.47) (stroke (width 0.12) (type solid)) (layer "F.SilkS"))
  (fp_line (start 7.8 -1.47) (end 2.36 -1.47) (stroke (width 0.12) (type solid)) (layer "F.SilkS"))
  (fp_line (start 7.8 1.47) (end 7.8 -1.47) (stroke (width 0.12) (type solid)) (layer "F.SilkS"))
  (fp_line (start 8.82 0) (end 7.8 0) (stroke (width 0.12) (type solid)) (layer "F.SilkS"))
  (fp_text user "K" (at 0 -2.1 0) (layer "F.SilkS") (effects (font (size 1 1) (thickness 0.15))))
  (pad "1" thru_hole rect (at 0 0) (size 2.2 2.2) (drill 1.1) (layers "*.Cu" "*.Mask") (remove_unused_layers no) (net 1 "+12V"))
  (pad "2" thru_hole oval (at 10.16 0) (size 2.2 2.2) (drill 1.1) (layers "*.Cu" "*.Mask") (remove_unused_layers no) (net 4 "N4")))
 (gr_rect (start 100 50) (end 166.5 115) (stroke (width 0.05) (type default)) (fill no) (layer "Edge.Cuts"))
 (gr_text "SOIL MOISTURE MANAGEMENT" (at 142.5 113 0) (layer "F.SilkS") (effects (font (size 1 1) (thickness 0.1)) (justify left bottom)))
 (segment (start 143 70.66) (end 143 70.5) (width 0.2) (layer "F.Cu") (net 6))
 (segment (start 105 88.5) (end 106.101 87.399) (width 0.2) (layer "F.Cu") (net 6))
 (segment (start 124.101 87.399) (end 126 85.5) (width 0.2) (layer "F.Cu") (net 6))
 (segment (start 106.101 87.399) (end 124.101 87.399) (width 0.2) (layer "F.Cu") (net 6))
 (segment (start 145.54 73.2) (end 143 70.66) (width 0.2) (layer "F.Cu") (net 6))
 (via (at 126 85.5) (size 0.6) (drill 0.3) (layers "F.Cu" "B.Cu") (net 6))
 (via (at 143 70.5) (size 0.6) (drill 0.3) (layers "F.Cu" "B.Cu") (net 6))
 (segment (start 126 85.5) (end 141 70.5) (width 0.2) (layer "B.Cu") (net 6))
 (segment (start 141 70.5) (end 143 70.5) (width 0.2) (layer "B.Cu") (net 6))
 (segment (start 117.24 73.26) (end 120.24 73.26) (width 0.2) (layer "F.Cu") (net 2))
 (segment (start 138.5 90.73) (end 138.5 89.5) (width 0.2) (layer "F.Cu") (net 2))
 (segment (start 142 86.265) (end 144 88.265) (width 0.2) (layer "F.Cu") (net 2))
 (segment (start 114.66 78.34) (end 116 77) (width 0.2) (layer "F.Cu") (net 2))
 (segment (start 135.27 87.27) (end 121.26 73.26) (width 0.2) (layer "F.Cu") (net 2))
 (segment (start 145.54 69.15) (end 142.85 69.15) (width 0.2) (layer "F.Cu") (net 2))
 (segment (start 135.27 87.5) (end 138.5 90.73) (width 0.2) (layer "F.Cu") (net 2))
 (segment (start 121.26 73.26) (end 120.24 73.26) (width 0.2) (layer "F.Cu") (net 2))
 (segment (start 139.735 88.265) (end 144 88.265) (width 0.2) (layer "F.Cu") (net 2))
 (segment (start 154 87) (end 152.735 88.265) (width 0.2) (layer "F.Cu") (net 2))
 (segment (start 135.27 87.5) (end 135.27 87.27) (width 0.2) (layer "F.Cu") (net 2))
 (segment (start 142 70) (end 142 86.265) (width 0.2) (layer "F.Cu") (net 2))
 (segment (start 105 78.34) (end 114.66 78.34) (width 0.2) (layer "F.Cu") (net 2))
 (segment (start 142.85 69.15) (end 142 70) (width 0.2) (layer "F.Cu") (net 2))
 (segment (start 116 74.5) (end 117.24 73.26) (width 0.2) (layer "F.Cu") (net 2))
 (segment (start 138 105.5) (end 135 105.5) (width 0.2) (layer "F.Cu") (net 2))
 (segment (start 116 77) (end 116 74.5) (width 0.2) (layer "F.Cu") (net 2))
 (segment (start 152.735 88.265) (end 144 88.265) (width 0.2) (layer "F.Cu") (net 2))
 (segment (start 138.5 90.73) (end 138.5 105) (width 0.2) (layer "F.Cu") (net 2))
 (segment (start 138.5 89.5) (end 139.735 88.265) (width 0.2) (layer "F.Cu") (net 2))
 (segment (start 138.5 105) (end 138 105.5) (width 0.2) (layer "F.Cu") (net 2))
 (segment (start 125 100) (end 123.66 98.66) (width 0.2) (layer "F.Cu") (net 3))
 (segment (start 126.04 108.04) (end 125 107) (width 0.2) (layer "F.Cu") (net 3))
 (segment (start 123.66 98.66) (end 120.24 98.66) (width 0.2) (layer "F.Cu") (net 3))
 (segment (start 135 108.04) (end 126.04 108.04) (width 0.2) (layer "F.Cu") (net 3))
 (segment (start 125 107) (end 125 100) (width 0.2) (layer "F.Cu") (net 3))
 (segment (start 124.671 79.441) (end 124.5 79.27) (width 0.2) (layer "F.Cu") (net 4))
 (segment (start 124.671 79.441) (end 132.73 87.5) (width 0.2) (layer "F.Cu") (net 4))
 (segment (start 102 57) (end 101.5 57.5) (width 0.2) (layer "F.Cu") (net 4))
 (segment (start 104.54395 79.441) (end 124.671 79.441) (width 0.2) (layer "F.Cu") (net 4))
 (segment (start 153.58 62.92) (end 153.58 58.5) (width 0.2) (layer "F.Cu") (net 4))
 (segment (start 153 63.5) (end 153.58 62.92) (width 0.2) (layer "F.Cu") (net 4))
 (segment (start 101.5 57.5) (end 101.5 76.39705) (width 0.2) (layer "F.Cu") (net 4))
 (segment (start 101.5 76.39705) (end 104.54395 79.441) (width 0.2) (layer "F.Cu") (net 4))
 (segment (start 104.5 57) (end 102 57) (width 0.2) (layer "F.Cu") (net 4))
 (segment (start 124.5 79.27) (end 124.5 77.5) (width 0.2) (layer "F.Cu") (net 4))
 (via (at 124.5 77.5) (size 0.6) (drill 0.3) (layers "F.Cu" "B.Cu") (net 4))
 (via (at 153 63.5) (size 0.6) (drill 0.3) (layers "F.Cu" "B.Cu") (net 4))
 (segment (start 151.5 65) (end 153 63.5) (width 0.2) (layer "B.Cu") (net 4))
 (segment (start 126 65) (end 151.5 65) (width 0.2) (layer "B.Cu") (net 4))
 (segment (start 124.5 77.5) (end 124.5 66.5) (width 0.2) (layer "B.Cu") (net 4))
 (segment (start 124.5 66.5) (end 126 65) (width 0.2) (layer "B.Cu") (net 4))
 (segment (start 139.92 55) (end 113 55) (width 0.2) (layer "F.Cu") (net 1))
 (segment (start 134 87.5) (end 134 101.96) (width 0.2) (layer "F.Cu") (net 1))
 (segment (start 143.42 59.41) (end 143.42 58.5) (width 0.2) (layer "F.Cu") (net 1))
 (segment (start 144 85.725) (end 147.775 85.725) (width 0.2) (layer "F.Cu") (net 1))
 (segment (start 113 55) (end 110.25 55) (width 0.2) (layer "F.Cu") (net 1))
 (segment (start 122.5 55) (end 113 55) (width 0.2) (layer "F.Cu") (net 1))
 (segment (start 134 89.5) (end 131 92.5) (width 0.2) (layer "F.Cu") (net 1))
 (segment (start 143.42 58.5) (end 139.92 55) (width 0.2) (layer "F.Cu") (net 1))
 (segment (start 124.5 57) (end 122.5 55) (width 0.2) (layer "F.Cu") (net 1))
 (segment (start 110.25 55) (end 108.25 57) (width 0.2) (layer "F.Cu") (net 1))
 (segment (start 134 101.96) (end 135 102.96) (width 0.2) (layer "F.Cu") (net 1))
 (segment (start 153.16 73.2) (end 153.16 69.15) (width 0.2) (layer "F.Cu") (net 1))
 (segment (start 147.775 85.725) (end 153.16 80.34) (width 0.2) (layer "F.Cu") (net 1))
 (segment (start 144 85.725) (end 144 83) (width 0.2) (layer "F.Cu") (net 1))
 (segment (start 144 83) (end 143.5 82.5) (width 0.2) (layer "F.Cu") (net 1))
 (segment (start 153.16 80.34) (end 153.16 73.2) (width 0.2) (layer "F.Cu") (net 1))
 (segment (start 134 87.5) (end 134 89.5) (width 0.2) (layer "F.Cu") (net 1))
 (segment (start 153.16 69.15) (end 143.42 59.41) (width 0.2) (layer "F.Cu") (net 1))
 (via (at 131 92.5) (size 0.6) (drill 0.3) (layers "F.Cu" "B.Cu") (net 1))
 (via (at 143.5 82.5) (size 0.6) (drill 0.3) (layers "F.Cu" "B.Cu") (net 1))
 (segment (start 143.5 82.5) (end 141.5 82.5) (width 0.2) (layer "B.Cu") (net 1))
 (segment (start 132 93.5) (end 139.5 93.5) (width 0.2) (layer "B.Cu") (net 1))
 (segment (start 141.5 82.5) (end 140.5 83.5) (width 0.2) (layer "B.Cu") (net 1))
 (segment (start 132 93.5) (end 131 92.5) (width 0.2) (layer "B.Cu") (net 1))
 (segment (start 139.5 93.5) (end 140.5 92.5) (width 0.2) (layer "B.Cu") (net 1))
 (segment (start 140.5 92.5) (end 140.5 83.5) (width 0.2) (layer "B.Cu") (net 1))
 (segment (start 127.999 58.501) (end 107.149 58.501) (width 0.2) (layer "F.Cu") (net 5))
 (segment (start 160 84.5) (end 159.96 84.46) (width 0.2) (layer "F.Cu") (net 5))
 (segment (start 157.099 54.599) (end 161 58.5) (width 0.2) (layer "F.Cu") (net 5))
 (segment (start 161 83.5) (end 160 84.5) (width 0.2) (layer "F.Cu") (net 5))
 (segment (start 106.949 58.301) (end 106.949 55.699) (width 0.2) (layer "F.Cu") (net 5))
 (segment (start 129.5 57) (end 127.999 58.501) (width 0.2) (layer "F.Cu") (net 5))
 (segment (start 108.049 54.599) (end 157.099 54.599) (width 0.2) (layer "F.Cu") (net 5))
 (segment (start 159.96 84.46) (end 154 84.46) (width 0.2) (layer "F.Cu") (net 5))
 (segment (start 107.149 58.501) (end 106.949 58.301) (width 0.2) (layer "F.Cu") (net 5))
 (segment (start 161 58.5) (end 161 83.5) (width 0.2) (layer "F.Cu") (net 5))
 (segment (start 106.949 55.699) (end 108.049 54.599) (width 0.2) (layer "F.Cu") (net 5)))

